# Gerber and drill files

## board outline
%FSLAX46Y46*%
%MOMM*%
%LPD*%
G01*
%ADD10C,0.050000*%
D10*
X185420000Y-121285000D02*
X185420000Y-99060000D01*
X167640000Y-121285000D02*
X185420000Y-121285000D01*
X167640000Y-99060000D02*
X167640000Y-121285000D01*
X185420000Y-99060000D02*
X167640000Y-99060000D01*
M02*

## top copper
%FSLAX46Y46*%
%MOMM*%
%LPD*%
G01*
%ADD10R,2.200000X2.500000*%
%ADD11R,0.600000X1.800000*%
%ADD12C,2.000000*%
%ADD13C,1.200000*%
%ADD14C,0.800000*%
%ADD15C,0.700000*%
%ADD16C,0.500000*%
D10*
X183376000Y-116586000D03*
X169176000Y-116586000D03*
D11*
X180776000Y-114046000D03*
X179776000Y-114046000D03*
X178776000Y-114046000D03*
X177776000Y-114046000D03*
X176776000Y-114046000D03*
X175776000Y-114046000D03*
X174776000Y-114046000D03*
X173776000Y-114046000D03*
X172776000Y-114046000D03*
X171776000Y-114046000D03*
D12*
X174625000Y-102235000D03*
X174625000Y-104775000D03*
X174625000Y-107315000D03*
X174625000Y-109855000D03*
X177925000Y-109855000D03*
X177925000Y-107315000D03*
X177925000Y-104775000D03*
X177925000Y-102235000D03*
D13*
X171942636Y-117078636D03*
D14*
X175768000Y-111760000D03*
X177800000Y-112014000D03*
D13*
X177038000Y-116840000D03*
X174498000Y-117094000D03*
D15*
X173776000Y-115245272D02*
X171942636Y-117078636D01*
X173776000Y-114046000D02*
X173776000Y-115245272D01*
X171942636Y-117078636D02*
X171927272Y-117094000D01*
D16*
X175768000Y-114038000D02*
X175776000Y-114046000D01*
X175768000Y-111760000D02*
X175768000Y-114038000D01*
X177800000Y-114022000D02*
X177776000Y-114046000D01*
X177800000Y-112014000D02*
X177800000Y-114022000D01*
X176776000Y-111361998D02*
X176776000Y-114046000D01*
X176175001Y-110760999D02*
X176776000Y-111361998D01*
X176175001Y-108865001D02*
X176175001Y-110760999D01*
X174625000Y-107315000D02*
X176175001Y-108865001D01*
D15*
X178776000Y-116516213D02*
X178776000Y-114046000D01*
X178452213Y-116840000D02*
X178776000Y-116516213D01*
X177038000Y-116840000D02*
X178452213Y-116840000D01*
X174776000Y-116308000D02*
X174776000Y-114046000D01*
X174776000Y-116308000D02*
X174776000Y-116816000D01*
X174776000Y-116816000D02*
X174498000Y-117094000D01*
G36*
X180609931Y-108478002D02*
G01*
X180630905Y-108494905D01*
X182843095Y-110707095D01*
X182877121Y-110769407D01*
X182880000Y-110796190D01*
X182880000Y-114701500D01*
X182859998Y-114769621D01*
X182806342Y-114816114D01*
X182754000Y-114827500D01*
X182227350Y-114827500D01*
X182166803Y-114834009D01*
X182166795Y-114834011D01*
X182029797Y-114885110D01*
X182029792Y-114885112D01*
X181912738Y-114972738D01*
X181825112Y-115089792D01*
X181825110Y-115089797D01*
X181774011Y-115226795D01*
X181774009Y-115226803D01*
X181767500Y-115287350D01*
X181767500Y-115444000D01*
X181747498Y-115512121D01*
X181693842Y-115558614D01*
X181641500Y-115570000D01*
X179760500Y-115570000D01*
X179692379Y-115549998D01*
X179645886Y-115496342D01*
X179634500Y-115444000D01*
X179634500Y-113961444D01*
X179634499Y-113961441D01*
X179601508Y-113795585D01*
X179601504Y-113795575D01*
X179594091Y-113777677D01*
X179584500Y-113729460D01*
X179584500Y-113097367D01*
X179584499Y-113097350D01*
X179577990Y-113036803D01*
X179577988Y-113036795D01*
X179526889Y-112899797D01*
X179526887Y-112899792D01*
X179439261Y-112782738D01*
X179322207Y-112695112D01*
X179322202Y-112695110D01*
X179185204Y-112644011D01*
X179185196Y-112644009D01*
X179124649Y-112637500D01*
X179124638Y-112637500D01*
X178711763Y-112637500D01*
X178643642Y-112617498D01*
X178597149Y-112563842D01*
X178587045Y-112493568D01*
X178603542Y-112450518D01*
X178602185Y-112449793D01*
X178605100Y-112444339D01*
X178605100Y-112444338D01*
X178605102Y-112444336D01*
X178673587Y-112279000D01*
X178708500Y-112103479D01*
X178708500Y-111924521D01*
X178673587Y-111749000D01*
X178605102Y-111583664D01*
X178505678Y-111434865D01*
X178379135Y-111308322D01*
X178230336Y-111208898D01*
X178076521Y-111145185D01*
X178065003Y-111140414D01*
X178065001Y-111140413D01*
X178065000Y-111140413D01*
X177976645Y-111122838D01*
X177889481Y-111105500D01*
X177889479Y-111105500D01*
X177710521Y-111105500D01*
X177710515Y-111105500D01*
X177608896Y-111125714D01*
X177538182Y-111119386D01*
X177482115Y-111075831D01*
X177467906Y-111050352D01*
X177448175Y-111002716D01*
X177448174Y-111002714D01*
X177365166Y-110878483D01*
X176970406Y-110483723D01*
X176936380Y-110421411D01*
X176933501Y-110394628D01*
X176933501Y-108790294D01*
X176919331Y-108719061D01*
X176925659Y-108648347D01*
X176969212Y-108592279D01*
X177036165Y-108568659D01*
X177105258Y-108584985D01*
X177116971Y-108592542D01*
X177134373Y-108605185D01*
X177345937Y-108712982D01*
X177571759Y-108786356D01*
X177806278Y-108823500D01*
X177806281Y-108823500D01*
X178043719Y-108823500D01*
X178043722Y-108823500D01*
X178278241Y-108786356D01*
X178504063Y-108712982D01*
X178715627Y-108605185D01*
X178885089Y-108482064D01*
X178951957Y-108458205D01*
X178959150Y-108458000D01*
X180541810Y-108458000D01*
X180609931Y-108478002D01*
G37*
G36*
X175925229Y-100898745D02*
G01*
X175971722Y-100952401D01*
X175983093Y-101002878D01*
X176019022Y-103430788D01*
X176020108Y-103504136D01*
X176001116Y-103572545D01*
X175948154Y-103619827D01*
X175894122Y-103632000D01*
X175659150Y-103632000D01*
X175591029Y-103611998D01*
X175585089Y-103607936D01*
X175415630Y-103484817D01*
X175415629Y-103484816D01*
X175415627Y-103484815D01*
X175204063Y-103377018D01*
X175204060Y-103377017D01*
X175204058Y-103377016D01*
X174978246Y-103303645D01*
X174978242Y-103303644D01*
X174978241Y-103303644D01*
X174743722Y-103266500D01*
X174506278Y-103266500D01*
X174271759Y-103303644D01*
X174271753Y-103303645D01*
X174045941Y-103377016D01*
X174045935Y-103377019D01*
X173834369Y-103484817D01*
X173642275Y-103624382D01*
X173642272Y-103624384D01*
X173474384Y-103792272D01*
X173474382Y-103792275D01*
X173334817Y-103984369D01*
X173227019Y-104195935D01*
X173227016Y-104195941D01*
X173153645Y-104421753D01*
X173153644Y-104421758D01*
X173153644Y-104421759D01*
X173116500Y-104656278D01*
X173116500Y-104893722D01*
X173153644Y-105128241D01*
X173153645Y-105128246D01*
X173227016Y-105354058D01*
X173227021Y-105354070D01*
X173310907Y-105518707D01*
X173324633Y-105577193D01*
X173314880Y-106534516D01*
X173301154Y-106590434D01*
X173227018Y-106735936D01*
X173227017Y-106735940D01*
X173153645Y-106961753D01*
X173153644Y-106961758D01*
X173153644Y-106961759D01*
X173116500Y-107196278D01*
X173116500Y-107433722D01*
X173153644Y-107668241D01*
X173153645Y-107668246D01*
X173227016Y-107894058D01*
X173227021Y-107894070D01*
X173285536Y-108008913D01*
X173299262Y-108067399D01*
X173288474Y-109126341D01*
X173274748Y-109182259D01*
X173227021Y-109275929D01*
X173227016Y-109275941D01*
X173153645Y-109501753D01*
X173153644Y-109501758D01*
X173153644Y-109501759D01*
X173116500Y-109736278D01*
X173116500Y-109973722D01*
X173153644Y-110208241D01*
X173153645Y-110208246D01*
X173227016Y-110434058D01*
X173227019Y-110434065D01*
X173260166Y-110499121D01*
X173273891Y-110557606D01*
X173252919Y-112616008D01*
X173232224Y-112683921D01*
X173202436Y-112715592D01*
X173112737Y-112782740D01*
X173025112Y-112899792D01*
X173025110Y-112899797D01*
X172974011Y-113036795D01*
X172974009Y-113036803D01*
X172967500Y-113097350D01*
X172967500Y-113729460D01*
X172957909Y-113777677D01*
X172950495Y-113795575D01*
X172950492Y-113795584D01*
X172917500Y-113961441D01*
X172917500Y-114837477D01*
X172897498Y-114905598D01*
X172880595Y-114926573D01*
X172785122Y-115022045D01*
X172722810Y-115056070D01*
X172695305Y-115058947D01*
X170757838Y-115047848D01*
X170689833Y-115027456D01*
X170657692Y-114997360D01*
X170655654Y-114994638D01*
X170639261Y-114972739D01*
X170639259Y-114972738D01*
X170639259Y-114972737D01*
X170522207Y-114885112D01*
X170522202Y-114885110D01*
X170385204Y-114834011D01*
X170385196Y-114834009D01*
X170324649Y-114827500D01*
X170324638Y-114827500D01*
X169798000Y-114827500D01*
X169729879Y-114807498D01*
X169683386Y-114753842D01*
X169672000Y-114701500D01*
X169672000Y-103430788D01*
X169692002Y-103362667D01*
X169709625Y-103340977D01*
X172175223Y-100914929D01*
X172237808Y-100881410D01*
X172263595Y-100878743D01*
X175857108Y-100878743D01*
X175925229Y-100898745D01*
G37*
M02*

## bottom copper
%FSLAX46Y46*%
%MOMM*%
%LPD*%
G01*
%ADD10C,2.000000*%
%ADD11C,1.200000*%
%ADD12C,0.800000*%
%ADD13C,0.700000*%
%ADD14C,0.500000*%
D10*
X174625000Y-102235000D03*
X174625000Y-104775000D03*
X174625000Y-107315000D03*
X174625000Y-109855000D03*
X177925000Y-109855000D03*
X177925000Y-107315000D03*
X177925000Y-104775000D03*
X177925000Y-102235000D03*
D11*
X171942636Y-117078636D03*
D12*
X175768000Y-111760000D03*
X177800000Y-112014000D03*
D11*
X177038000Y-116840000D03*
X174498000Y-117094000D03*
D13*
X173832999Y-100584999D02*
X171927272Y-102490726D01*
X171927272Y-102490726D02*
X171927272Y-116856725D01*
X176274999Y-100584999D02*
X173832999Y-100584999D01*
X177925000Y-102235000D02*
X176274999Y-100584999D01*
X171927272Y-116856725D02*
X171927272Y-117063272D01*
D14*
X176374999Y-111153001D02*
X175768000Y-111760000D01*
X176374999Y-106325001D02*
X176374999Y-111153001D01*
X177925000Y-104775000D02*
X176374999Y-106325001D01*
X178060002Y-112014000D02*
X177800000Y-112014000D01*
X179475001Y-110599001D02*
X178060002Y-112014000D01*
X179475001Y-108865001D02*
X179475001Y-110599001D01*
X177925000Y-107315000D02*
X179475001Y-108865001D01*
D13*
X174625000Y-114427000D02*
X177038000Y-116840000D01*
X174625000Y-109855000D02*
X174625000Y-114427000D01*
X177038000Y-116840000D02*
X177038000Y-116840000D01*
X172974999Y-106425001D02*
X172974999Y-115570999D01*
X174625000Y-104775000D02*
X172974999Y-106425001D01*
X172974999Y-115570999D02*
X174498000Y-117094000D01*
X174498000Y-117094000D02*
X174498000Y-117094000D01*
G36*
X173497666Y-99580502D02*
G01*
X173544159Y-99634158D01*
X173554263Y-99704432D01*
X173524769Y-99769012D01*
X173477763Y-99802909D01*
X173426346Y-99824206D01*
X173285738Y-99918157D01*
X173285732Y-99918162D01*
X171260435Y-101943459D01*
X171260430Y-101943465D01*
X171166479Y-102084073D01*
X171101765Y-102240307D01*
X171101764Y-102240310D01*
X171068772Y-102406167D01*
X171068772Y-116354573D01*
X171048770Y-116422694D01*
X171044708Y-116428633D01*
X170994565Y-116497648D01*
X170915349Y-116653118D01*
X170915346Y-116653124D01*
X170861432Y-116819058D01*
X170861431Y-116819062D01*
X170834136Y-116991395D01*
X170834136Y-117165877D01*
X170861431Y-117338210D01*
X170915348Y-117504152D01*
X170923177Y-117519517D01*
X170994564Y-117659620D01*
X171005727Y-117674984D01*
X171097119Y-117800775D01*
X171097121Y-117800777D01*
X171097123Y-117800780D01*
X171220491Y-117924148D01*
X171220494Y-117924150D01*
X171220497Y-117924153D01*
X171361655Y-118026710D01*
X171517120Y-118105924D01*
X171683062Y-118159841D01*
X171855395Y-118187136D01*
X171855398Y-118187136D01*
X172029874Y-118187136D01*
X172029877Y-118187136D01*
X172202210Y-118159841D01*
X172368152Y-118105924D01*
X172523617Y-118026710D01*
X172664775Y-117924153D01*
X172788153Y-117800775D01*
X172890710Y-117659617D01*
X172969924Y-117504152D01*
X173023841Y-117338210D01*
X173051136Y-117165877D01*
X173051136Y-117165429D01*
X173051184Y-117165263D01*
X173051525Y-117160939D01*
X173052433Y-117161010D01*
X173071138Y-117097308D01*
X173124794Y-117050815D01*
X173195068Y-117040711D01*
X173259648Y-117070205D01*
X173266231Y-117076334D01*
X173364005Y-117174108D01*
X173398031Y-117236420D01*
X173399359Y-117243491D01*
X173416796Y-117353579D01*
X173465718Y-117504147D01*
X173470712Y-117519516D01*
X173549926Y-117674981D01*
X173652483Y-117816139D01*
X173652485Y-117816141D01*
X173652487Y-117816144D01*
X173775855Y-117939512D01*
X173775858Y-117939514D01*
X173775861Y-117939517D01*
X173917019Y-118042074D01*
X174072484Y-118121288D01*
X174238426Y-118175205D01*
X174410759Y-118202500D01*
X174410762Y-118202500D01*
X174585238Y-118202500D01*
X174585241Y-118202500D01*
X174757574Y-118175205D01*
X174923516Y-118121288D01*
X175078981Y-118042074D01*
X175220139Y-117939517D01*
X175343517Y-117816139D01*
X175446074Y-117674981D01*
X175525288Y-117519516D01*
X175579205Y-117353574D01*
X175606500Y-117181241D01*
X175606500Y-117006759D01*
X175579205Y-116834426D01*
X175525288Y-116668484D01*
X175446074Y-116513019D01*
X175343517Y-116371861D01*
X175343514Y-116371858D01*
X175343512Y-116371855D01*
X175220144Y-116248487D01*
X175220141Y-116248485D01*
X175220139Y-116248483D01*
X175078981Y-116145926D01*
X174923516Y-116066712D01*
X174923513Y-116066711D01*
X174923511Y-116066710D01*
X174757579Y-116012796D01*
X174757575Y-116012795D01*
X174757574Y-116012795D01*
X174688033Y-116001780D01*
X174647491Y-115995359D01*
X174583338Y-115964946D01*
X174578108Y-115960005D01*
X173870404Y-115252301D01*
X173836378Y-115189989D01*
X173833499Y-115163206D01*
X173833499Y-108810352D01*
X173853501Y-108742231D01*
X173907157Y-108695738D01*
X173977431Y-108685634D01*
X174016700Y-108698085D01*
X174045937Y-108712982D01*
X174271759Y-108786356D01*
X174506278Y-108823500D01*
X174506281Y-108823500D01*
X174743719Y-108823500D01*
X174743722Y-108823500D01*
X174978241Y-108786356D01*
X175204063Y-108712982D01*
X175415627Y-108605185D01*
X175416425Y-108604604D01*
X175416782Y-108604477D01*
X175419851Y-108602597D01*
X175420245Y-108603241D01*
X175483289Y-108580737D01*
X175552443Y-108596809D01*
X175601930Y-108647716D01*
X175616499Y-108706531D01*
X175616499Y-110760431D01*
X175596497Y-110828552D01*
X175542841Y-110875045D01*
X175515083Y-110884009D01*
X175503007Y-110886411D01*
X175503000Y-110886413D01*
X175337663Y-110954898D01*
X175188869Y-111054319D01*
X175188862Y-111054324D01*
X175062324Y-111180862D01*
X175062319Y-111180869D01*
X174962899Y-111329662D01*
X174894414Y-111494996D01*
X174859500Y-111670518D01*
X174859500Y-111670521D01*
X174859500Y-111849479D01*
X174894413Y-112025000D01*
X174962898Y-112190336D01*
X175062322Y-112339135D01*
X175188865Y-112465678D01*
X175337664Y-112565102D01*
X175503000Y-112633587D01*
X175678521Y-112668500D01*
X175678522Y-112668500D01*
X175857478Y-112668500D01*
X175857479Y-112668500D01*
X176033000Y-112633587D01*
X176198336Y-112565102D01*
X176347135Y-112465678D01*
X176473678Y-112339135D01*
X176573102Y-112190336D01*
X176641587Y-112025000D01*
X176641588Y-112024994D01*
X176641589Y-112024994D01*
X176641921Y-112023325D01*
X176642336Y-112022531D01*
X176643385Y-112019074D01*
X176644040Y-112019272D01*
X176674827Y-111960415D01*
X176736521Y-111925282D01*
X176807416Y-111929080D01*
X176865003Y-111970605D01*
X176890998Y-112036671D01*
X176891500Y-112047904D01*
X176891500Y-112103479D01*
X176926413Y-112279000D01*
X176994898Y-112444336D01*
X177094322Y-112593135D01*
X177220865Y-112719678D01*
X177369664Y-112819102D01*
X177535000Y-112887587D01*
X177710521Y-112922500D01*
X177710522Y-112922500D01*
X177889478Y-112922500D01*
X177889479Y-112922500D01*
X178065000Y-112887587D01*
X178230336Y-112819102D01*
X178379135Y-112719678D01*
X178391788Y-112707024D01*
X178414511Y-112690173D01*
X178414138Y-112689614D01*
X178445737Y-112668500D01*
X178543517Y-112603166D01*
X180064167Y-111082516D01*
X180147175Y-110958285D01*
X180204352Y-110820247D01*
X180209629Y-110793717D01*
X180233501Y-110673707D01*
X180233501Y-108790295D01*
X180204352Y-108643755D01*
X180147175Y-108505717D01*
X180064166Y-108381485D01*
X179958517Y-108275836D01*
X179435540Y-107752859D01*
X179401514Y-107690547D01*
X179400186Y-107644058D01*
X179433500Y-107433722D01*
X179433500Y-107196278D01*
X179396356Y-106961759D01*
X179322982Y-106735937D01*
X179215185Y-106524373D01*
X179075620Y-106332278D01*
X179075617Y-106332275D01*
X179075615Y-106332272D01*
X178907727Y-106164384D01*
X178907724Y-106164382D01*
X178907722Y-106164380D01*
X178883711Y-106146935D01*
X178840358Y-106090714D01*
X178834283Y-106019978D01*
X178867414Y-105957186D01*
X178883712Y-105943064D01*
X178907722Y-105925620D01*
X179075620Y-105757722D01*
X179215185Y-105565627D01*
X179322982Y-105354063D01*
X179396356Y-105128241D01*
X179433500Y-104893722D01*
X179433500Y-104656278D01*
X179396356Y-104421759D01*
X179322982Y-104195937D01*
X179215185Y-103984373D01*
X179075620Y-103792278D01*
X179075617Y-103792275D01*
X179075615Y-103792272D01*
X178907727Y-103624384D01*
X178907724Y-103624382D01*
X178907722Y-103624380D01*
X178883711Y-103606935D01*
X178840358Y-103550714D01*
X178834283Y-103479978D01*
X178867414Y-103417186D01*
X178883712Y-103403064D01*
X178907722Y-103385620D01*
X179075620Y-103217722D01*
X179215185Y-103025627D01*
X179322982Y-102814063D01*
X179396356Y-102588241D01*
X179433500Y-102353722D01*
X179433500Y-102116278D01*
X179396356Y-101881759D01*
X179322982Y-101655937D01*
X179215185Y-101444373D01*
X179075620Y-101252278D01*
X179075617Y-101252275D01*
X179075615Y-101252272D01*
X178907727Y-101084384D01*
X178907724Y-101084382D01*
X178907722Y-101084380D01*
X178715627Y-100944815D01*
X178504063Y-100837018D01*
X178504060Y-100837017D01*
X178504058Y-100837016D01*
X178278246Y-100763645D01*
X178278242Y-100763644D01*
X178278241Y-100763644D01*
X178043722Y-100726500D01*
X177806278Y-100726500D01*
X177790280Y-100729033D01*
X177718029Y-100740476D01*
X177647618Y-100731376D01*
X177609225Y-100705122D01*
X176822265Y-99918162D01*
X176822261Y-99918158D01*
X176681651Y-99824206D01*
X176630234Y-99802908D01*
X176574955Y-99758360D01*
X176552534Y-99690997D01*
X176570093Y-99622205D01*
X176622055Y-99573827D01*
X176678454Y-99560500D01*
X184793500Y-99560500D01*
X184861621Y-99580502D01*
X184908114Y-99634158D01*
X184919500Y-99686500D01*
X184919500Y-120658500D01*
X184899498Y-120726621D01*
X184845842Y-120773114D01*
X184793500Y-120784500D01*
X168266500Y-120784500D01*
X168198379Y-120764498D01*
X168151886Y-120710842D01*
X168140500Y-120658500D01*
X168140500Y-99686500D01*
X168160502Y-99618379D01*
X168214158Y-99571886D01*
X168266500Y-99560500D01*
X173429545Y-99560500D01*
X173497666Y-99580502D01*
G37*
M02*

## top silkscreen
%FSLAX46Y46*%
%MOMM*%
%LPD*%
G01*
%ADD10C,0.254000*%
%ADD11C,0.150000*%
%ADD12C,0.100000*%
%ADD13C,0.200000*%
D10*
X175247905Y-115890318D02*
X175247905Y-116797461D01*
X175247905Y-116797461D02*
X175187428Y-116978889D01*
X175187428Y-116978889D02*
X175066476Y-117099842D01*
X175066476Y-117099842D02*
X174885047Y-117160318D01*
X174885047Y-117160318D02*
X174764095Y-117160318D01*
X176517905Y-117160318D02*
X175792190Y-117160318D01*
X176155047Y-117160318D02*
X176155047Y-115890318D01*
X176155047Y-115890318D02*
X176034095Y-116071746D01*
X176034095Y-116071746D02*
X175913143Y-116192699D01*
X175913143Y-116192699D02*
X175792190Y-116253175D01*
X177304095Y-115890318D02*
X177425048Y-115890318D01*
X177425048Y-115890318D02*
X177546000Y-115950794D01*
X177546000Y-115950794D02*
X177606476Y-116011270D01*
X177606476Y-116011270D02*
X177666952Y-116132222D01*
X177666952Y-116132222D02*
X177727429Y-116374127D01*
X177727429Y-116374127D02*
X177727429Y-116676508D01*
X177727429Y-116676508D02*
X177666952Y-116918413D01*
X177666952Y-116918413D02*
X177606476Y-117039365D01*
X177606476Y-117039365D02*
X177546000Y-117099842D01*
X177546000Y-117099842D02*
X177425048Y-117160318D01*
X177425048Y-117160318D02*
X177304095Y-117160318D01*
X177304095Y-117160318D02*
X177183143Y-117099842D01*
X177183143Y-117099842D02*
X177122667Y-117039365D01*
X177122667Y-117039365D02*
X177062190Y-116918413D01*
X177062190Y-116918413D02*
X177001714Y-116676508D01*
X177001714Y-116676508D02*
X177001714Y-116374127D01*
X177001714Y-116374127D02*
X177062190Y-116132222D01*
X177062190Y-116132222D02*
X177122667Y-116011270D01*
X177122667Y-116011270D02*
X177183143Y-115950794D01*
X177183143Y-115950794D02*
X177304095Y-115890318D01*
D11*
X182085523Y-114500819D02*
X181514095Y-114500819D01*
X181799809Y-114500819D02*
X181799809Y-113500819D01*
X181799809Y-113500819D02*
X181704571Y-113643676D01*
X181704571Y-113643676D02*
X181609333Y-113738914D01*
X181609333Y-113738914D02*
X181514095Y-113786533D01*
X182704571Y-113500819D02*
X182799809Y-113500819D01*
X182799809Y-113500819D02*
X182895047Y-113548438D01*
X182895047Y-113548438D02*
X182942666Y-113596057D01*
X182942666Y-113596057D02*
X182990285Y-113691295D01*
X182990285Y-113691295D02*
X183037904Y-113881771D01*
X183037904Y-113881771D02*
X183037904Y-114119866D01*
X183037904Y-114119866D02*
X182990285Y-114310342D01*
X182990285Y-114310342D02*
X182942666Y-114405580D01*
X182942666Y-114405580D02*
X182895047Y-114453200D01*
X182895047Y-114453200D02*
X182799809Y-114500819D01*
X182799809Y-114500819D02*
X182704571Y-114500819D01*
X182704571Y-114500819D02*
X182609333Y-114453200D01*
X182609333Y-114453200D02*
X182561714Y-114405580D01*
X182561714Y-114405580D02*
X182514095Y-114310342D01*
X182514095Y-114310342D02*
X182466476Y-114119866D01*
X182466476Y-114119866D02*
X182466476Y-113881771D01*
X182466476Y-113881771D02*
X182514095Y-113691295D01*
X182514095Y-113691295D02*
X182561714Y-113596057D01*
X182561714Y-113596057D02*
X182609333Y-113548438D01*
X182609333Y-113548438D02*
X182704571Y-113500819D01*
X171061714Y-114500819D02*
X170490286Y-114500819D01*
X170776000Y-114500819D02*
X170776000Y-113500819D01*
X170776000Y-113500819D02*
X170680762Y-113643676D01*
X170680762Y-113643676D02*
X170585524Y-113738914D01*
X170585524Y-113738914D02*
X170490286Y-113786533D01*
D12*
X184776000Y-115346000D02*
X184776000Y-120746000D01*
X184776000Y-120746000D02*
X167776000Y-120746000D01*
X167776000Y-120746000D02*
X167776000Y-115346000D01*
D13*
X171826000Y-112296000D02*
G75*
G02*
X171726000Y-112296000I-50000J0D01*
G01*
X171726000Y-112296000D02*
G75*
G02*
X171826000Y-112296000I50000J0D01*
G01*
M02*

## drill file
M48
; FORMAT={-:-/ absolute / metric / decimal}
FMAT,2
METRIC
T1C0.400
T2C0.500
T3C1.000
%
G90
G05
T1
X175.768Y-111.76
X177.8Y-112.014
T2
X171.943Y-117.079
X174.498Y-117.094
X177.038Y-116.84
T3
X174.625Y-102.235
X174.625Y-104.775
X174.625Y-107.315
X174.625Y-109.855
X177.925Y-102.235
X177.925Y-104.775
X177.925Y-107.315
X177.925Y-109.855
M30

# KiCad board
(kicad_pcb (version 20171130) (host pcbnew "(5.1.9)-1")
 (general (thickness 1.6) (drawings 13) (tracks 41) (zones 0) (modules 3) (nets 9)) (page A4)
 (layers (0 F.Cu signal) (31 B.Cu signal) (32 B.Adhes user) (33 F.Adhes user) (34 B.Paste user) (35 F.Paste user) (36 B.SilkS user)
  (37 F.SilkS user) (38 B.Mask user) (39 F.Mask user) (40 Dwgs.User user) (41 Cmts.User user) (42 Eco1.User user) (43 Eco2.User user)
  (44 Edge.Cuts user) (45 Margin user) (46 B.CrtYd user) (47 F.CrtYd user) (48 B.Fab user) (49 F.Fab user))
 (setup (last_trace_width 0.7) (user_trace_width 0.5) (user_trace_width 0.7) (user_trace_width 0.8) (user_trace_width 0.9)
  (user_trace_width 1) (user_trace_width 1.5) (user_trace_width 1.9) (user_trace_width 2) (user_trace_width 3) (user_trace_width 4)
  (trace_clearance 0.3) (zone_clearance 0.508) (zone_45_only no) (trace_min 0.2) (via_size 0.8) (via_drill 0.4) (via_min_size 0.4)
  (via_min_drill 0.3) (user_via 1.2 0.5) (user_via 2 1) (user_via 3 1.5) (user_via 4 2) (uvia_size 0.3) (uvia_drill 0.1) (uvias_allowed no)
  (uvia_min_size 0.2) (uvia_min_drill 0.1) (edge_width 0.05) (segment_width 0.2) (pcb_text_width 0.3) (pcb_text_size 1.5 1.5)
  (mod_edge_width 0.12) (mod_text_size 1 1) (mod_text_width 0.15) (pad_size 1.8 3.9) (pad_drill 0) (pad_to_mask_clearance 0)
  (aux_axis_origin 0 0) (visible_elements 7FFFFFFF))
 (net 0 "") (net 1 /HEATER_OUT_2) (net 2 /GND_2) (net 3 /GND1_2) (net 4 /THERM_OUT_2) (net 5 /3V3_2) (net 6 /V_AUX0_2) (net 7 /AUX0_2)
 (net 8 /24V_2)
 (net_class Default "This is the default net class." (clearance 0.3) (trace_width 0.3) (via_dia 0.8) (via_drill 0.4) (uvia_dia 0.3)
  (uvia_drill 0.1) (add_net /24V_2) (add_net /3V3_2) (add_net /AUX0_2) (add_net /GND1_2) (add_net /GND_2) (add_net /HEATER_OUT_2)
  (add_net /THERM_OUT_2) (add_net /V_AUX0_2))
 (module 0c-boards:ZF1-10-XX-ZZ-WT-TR (layer F.Cu) (at 176.276 114.046)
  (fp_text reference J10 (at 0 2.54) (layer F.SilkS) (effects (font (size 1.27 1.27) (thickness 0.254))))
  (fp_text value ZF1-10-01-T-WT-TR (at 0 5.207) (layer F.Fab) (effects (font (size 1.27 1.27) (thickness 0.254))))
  (fp_line (start 8.5 1.3) (end 8.5 6.7) (layer F.SilkS) (width 0.1))
  (fp_line (start 8.5 6.7) (end -8.5 6.7) (layer F.SilkS) (width 0.1))
  (fp_line (start -8.5 6.7) (end -8.5 1.3) (layer F.SilkS) (width 0.1))
  (fp_circle (center -4.5 -1.75) (end -4.5 -1.7) (layer F.SilkS) (width 0.2))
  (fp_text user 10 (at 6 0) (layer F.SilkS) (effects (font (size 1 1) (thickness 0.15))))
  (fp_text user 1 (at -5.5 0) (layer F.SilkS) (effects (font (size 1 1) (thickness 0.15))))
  (pad 12 smd rect (at 7.1 2.54) (size 2.2 2.5) (layers F.Cu F.Paste F.Mask))
  (pad 11 smd rect (at -7.1 2.54) (size 2.2 2.5) (layers F.Cu F.Paste F.Mask))
  (pad 10 smd rect (at 4.5 0) (size 0.6 1.8) (layers F.Cu F.Paste F.Mask) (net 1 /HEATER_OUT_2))
  (pad 9 smd rect (at 3.5 0) (size 0.6 1.8) (layers F.Cu F.Paste F.Mask) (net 1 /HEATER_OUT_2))
  (pad 8 smd rect (at 2.5 0) (size 0.6 1.8) (layers F.Cu F.Paste F.Mask) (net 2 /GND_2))
  (pad 7 smd rect (at 1.5 0) (size 0.6 1.8) (layers F.Cu F.Paste F.Mask) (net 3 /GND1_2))
  (pad 6 smd rect (at 0.5 0) (size 0.6 1.8) (layers F.Cu F.Paste F.Mask) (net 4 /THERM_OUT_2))
  (pad 5 smd rect (at -0.5 0) (size 0.6 1.8) (layers F.Cu F.Paste F.Mask) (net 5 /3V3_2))
  (pad 4 smd rect (at -1.5 0) (size 0.6 1.8) (layers F.Cu F.Paste F.Mask) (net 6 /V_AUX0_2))
  (pad 3 smd rect (at -2.5 0) (size 0.6 1.8) (layers F.Cu F.Paste F.Mask) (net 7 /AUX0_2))
  (pad 2 smd rect (at -3.5 0) (size 0.6 1.8) (layers F.Cu F.Paste F.Mask) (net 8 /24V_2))
  (pad 1 smd rect (at -4.5 0) (size 0.6 1.8) (layers F.Cu F.Paste F.Mask) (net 8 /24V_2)))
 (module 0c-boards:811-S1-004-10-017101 (layer B.Cu) (at 174.625 106.045 270)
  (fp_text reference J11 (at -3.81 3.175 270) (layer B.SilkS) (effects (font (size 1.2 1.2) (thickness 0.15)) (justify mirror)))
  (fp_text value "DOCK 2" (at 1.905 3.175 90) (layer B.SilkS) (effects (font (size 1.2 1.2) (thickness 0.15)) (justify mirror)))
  (pad 1 thru_hole circle (at -3.81 0 270) (size 2 2) (drill 1) (layers *.Cu *.Mask) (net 8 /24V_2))
  (pad 2 thru_hole circle (at -1.27 0 270) (size 2 2) (drill 1) (layers *.Cu *.Mask) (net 6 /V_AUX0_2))
  (pad 3 thru_hole circle (at 1.27 0 270) (size 2 2) (drill 1) (layers *.Cu *.Mask) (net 4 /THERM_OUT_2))
  (pad 4 thru_hole circle (at 3.81 0 270) (size 2 2) (drill 1) (layers *.Cu *.Mask) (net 2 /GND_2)))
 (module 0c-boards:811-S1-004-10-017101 (layer B.Cu) (at 177.925 106.045 90)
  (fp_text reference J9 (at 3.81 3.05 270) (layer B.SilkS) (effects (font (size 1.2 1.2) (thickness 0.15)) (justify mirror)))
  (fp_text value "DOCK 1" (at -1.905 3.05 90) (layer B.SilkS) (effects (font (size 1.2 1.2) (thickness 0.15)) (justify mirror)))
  (pad 1 thru_hole circle (at -3.81 0 90) (size 2 2) (drill 1) (layers *.Cu *.Mask) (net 1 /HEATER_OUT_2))
  (pad 2 thru_hole circle (at -1.27 0 90) (size 2 2) (drill 1) (layers *.Cu *.Mask) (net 3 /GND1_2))
  (pad 3 thru_hole circle (at 1.27 0 90) (size 2 2) (drill 1) (layers *.Cu *.Mask) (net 5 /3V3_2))
  (pad 4 thru_hole circle (at 3.81 0 90) (size 2 2) (drill 1) (layers *.Cu *.Mask) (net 7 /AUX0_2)))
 (gr_line (start 185.42 121.285) (end 185.42 99.06) (layer Edge.Cuts) (width 0.05))
 (gr_line (start 167.64 121.285) (end 185.42 121.285) (layer Edge.Cuts) (width 0.05))
 (gr_line (start 167.64 99.06) (end 167.64 121.285) (layer Edge.Cuts) (width 0.05))
 (gr_line (start 185.42 99.06) (end 167.64 99.06) (layer Edge.Cuts) (width 0.05))
 (segment (start 173.832999 100.584999) (end 171.927272 102.490726) (width 0.7) (layer B.Cu) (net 7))
 (segment (start 171.927272 102.490726) (end 171.927272 116.856725) (width 0.7) (layer B.Cu) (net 7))
 (segment (start 176.274999 100.584999) (end 173.832999 100.584999) (width 0.7) (layer B.Cu) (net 7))
 (segment (start 177.925 102.235) (end 176.274999 100.584999) (width 0.7) (layer B.Cu) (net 7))
 (segment (start 173.776 115.245272) (end 171.942636 117.078636) (width 0.7) (layer F.Cu) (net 7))
 (segment (start 173.776 114.046) (end 173.776 115.245272) (width 0.7) (layer F.Cu) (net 7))
 (segment (start 171.927272 116.856725) (end 171.927272 117.063272) (width 0.7) (layer B.Cu) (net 7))
 (segment (start 171.942636 117.078636) (end 171.927272 117.094) (width 0.7) (layer F.Cu) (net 7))
 (via (at 171.942636 117.078636) (size 1.2) (drill 0.5) (layers F.Cu B.Cu) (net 7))
 (via (at 175.768 111.76) (size 0.8) (drill 0.4) (layers F.Cu B.Cu) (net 5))
 (segment (start 176.374999 111.153001) (end 175.768 111.76) (width 0.5) (layer B.Cu) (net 5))
 (segment (start 176.374999 106.325001) (end 176.374999 111.153001) (width 0.5) (layer B.Cu) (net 5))
 (segment (start 177.925 104.775) (end 176.374999 106.325001) (width 0.5) (layer B.Cu) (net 5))
 (segment (start 175.768 114.038) (end 175.776 114.046) (width 0.5) (layer F.Cu) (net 5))
 (segment (start 175.768 111.76) (end 175.768 114.038) (width 0.5) (layer F.Cu) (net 5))
 (via (at 177.8 112.014) (size 0.8) (drill 0.4) (layers F.Cu B.Cu) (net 3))
 (segment (start 178.060002 112.014) (end 177.8 112.014) (width 0.5) (layer B.Cu) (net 3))
 (segment (start 179.475001 110.599001) (end 178.060002 112.014) (width 0.5) (layer B.Cu) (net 3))
 (segment (start 179.475001 108.865001) (end 179.475001 110.599001) (width 0.5) (layer B.Cu) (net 3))
 (segment (start 177.925 107.315) (end 179.475001 108.865001) (width 0.5) (layer B.Cu) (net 3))
 (segment (start 177.8 114.022) (end 177.776 114.046) (width 0.5) (layer F.Cu) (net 3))
 (segment (start 177.8 112.014) (end 177.8 114.022) (width 0.5) (layer F.Cu) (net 3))
 (segment (start 176.776 111.361998) (end 176.776 114.046) (width 0.5) (layer F.Cu) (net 4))
 (segment (start 176.175001 110.760999) (end 176.776 111.361998) (width 0.5) (layer F.Cu) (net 4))
 (segment (start 176.175001 108.865001) (end 176.175001 110.760999) (width 0.5) (layer F.Cu) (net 4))
 (segment (start 174.625 107.315) (end 176.175001 108.865001) (width 0.5) (layer F.Cu) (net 4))
 (segment (start 174.625 114.427) (end 177.038 116.84) (width 0.7) (layer B.Cu) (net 2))
 (segment (start 174.625 109.855) (end 174.625 114.427) (width 0.7) (layer B.Cu) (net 2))
 (segment (start 178.776 116.516213) (end 178.776 114.046) (width 0.7) (layer F.Cu) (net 2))
 (segment (start 178.452213 116.84) (end 178.776 116.516213) (width 0.7) (layer F.Cu) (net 2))
 (segment (start 177.038 116.84) (end 178.452213 116.84) (width 0.7) (layer F.Cu) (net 2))
 (segment (start 177.038 116.84) (end 177.038 116.84) (width 0.7) (layer B.Cu) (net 2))
 (via (at 177.038 116.84) (size 1.2) (drill 0.5) (layers F.Cu B.Cu) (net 2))
 (segment (start 172.974999 106.425001) (end 172.974999 115.570999) (width 0.7) (layer B.Cu) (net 6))
 (segment (start 174.625 104.775) (end 172.974999 106.425001) (width 0.7) (layer B.Cu) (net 6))
 (segment (start 174.776 116.308) (end 174.776 114.046) (width 0.7) (layer F.Cu) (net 6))
 (segment (start 172.974999 115.570999) (end 174.498 117.094) (width 0.7) (layer B.Cu) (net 6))
 (segment (start 174.776 116.308) (end 174.776 116.816) (width 0.7) (layer F.Cu) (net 6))
 (segment (start 174.776 116.816) (end 174.498 117.094) (width 0.7) (layer F.Cu) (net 6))
 (segment (start 174.498 117.094) (end 174.498 117.094) (width 0.7) (layer B.Cu) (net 6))
 (via (at 174.498 117.094) (size 1.2) (drill 0.5) (layers F.Cu B.Cu) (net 6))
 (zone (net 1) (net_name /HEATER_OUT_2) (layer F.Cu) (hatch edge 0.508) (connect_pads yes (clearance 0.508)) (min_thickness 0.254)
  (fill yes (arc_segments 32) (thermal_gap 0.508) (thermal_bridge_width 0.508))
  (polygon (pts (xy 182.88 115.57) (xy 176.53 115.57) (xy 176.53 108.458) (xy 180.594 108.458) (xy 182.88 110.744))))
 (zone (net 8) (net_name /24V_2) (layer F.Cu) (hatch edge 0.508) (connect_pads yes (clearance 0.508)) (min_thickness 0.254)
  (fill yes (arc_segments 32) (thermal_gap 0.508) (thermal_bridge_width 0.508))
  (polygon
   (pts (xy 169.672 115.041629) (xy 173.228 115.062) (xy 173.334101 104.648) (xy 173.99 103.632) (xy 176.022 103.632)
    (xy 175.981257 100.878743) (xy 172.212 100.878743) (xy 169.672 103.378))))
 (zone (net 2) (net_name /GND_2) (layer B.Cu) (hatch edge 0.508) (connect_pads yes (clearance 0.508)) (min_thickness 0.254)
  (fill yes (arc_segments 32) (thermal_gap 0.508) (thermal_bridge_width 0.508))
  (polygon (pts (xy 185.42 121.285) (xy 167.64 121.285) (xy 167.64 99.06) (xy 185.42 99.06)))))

